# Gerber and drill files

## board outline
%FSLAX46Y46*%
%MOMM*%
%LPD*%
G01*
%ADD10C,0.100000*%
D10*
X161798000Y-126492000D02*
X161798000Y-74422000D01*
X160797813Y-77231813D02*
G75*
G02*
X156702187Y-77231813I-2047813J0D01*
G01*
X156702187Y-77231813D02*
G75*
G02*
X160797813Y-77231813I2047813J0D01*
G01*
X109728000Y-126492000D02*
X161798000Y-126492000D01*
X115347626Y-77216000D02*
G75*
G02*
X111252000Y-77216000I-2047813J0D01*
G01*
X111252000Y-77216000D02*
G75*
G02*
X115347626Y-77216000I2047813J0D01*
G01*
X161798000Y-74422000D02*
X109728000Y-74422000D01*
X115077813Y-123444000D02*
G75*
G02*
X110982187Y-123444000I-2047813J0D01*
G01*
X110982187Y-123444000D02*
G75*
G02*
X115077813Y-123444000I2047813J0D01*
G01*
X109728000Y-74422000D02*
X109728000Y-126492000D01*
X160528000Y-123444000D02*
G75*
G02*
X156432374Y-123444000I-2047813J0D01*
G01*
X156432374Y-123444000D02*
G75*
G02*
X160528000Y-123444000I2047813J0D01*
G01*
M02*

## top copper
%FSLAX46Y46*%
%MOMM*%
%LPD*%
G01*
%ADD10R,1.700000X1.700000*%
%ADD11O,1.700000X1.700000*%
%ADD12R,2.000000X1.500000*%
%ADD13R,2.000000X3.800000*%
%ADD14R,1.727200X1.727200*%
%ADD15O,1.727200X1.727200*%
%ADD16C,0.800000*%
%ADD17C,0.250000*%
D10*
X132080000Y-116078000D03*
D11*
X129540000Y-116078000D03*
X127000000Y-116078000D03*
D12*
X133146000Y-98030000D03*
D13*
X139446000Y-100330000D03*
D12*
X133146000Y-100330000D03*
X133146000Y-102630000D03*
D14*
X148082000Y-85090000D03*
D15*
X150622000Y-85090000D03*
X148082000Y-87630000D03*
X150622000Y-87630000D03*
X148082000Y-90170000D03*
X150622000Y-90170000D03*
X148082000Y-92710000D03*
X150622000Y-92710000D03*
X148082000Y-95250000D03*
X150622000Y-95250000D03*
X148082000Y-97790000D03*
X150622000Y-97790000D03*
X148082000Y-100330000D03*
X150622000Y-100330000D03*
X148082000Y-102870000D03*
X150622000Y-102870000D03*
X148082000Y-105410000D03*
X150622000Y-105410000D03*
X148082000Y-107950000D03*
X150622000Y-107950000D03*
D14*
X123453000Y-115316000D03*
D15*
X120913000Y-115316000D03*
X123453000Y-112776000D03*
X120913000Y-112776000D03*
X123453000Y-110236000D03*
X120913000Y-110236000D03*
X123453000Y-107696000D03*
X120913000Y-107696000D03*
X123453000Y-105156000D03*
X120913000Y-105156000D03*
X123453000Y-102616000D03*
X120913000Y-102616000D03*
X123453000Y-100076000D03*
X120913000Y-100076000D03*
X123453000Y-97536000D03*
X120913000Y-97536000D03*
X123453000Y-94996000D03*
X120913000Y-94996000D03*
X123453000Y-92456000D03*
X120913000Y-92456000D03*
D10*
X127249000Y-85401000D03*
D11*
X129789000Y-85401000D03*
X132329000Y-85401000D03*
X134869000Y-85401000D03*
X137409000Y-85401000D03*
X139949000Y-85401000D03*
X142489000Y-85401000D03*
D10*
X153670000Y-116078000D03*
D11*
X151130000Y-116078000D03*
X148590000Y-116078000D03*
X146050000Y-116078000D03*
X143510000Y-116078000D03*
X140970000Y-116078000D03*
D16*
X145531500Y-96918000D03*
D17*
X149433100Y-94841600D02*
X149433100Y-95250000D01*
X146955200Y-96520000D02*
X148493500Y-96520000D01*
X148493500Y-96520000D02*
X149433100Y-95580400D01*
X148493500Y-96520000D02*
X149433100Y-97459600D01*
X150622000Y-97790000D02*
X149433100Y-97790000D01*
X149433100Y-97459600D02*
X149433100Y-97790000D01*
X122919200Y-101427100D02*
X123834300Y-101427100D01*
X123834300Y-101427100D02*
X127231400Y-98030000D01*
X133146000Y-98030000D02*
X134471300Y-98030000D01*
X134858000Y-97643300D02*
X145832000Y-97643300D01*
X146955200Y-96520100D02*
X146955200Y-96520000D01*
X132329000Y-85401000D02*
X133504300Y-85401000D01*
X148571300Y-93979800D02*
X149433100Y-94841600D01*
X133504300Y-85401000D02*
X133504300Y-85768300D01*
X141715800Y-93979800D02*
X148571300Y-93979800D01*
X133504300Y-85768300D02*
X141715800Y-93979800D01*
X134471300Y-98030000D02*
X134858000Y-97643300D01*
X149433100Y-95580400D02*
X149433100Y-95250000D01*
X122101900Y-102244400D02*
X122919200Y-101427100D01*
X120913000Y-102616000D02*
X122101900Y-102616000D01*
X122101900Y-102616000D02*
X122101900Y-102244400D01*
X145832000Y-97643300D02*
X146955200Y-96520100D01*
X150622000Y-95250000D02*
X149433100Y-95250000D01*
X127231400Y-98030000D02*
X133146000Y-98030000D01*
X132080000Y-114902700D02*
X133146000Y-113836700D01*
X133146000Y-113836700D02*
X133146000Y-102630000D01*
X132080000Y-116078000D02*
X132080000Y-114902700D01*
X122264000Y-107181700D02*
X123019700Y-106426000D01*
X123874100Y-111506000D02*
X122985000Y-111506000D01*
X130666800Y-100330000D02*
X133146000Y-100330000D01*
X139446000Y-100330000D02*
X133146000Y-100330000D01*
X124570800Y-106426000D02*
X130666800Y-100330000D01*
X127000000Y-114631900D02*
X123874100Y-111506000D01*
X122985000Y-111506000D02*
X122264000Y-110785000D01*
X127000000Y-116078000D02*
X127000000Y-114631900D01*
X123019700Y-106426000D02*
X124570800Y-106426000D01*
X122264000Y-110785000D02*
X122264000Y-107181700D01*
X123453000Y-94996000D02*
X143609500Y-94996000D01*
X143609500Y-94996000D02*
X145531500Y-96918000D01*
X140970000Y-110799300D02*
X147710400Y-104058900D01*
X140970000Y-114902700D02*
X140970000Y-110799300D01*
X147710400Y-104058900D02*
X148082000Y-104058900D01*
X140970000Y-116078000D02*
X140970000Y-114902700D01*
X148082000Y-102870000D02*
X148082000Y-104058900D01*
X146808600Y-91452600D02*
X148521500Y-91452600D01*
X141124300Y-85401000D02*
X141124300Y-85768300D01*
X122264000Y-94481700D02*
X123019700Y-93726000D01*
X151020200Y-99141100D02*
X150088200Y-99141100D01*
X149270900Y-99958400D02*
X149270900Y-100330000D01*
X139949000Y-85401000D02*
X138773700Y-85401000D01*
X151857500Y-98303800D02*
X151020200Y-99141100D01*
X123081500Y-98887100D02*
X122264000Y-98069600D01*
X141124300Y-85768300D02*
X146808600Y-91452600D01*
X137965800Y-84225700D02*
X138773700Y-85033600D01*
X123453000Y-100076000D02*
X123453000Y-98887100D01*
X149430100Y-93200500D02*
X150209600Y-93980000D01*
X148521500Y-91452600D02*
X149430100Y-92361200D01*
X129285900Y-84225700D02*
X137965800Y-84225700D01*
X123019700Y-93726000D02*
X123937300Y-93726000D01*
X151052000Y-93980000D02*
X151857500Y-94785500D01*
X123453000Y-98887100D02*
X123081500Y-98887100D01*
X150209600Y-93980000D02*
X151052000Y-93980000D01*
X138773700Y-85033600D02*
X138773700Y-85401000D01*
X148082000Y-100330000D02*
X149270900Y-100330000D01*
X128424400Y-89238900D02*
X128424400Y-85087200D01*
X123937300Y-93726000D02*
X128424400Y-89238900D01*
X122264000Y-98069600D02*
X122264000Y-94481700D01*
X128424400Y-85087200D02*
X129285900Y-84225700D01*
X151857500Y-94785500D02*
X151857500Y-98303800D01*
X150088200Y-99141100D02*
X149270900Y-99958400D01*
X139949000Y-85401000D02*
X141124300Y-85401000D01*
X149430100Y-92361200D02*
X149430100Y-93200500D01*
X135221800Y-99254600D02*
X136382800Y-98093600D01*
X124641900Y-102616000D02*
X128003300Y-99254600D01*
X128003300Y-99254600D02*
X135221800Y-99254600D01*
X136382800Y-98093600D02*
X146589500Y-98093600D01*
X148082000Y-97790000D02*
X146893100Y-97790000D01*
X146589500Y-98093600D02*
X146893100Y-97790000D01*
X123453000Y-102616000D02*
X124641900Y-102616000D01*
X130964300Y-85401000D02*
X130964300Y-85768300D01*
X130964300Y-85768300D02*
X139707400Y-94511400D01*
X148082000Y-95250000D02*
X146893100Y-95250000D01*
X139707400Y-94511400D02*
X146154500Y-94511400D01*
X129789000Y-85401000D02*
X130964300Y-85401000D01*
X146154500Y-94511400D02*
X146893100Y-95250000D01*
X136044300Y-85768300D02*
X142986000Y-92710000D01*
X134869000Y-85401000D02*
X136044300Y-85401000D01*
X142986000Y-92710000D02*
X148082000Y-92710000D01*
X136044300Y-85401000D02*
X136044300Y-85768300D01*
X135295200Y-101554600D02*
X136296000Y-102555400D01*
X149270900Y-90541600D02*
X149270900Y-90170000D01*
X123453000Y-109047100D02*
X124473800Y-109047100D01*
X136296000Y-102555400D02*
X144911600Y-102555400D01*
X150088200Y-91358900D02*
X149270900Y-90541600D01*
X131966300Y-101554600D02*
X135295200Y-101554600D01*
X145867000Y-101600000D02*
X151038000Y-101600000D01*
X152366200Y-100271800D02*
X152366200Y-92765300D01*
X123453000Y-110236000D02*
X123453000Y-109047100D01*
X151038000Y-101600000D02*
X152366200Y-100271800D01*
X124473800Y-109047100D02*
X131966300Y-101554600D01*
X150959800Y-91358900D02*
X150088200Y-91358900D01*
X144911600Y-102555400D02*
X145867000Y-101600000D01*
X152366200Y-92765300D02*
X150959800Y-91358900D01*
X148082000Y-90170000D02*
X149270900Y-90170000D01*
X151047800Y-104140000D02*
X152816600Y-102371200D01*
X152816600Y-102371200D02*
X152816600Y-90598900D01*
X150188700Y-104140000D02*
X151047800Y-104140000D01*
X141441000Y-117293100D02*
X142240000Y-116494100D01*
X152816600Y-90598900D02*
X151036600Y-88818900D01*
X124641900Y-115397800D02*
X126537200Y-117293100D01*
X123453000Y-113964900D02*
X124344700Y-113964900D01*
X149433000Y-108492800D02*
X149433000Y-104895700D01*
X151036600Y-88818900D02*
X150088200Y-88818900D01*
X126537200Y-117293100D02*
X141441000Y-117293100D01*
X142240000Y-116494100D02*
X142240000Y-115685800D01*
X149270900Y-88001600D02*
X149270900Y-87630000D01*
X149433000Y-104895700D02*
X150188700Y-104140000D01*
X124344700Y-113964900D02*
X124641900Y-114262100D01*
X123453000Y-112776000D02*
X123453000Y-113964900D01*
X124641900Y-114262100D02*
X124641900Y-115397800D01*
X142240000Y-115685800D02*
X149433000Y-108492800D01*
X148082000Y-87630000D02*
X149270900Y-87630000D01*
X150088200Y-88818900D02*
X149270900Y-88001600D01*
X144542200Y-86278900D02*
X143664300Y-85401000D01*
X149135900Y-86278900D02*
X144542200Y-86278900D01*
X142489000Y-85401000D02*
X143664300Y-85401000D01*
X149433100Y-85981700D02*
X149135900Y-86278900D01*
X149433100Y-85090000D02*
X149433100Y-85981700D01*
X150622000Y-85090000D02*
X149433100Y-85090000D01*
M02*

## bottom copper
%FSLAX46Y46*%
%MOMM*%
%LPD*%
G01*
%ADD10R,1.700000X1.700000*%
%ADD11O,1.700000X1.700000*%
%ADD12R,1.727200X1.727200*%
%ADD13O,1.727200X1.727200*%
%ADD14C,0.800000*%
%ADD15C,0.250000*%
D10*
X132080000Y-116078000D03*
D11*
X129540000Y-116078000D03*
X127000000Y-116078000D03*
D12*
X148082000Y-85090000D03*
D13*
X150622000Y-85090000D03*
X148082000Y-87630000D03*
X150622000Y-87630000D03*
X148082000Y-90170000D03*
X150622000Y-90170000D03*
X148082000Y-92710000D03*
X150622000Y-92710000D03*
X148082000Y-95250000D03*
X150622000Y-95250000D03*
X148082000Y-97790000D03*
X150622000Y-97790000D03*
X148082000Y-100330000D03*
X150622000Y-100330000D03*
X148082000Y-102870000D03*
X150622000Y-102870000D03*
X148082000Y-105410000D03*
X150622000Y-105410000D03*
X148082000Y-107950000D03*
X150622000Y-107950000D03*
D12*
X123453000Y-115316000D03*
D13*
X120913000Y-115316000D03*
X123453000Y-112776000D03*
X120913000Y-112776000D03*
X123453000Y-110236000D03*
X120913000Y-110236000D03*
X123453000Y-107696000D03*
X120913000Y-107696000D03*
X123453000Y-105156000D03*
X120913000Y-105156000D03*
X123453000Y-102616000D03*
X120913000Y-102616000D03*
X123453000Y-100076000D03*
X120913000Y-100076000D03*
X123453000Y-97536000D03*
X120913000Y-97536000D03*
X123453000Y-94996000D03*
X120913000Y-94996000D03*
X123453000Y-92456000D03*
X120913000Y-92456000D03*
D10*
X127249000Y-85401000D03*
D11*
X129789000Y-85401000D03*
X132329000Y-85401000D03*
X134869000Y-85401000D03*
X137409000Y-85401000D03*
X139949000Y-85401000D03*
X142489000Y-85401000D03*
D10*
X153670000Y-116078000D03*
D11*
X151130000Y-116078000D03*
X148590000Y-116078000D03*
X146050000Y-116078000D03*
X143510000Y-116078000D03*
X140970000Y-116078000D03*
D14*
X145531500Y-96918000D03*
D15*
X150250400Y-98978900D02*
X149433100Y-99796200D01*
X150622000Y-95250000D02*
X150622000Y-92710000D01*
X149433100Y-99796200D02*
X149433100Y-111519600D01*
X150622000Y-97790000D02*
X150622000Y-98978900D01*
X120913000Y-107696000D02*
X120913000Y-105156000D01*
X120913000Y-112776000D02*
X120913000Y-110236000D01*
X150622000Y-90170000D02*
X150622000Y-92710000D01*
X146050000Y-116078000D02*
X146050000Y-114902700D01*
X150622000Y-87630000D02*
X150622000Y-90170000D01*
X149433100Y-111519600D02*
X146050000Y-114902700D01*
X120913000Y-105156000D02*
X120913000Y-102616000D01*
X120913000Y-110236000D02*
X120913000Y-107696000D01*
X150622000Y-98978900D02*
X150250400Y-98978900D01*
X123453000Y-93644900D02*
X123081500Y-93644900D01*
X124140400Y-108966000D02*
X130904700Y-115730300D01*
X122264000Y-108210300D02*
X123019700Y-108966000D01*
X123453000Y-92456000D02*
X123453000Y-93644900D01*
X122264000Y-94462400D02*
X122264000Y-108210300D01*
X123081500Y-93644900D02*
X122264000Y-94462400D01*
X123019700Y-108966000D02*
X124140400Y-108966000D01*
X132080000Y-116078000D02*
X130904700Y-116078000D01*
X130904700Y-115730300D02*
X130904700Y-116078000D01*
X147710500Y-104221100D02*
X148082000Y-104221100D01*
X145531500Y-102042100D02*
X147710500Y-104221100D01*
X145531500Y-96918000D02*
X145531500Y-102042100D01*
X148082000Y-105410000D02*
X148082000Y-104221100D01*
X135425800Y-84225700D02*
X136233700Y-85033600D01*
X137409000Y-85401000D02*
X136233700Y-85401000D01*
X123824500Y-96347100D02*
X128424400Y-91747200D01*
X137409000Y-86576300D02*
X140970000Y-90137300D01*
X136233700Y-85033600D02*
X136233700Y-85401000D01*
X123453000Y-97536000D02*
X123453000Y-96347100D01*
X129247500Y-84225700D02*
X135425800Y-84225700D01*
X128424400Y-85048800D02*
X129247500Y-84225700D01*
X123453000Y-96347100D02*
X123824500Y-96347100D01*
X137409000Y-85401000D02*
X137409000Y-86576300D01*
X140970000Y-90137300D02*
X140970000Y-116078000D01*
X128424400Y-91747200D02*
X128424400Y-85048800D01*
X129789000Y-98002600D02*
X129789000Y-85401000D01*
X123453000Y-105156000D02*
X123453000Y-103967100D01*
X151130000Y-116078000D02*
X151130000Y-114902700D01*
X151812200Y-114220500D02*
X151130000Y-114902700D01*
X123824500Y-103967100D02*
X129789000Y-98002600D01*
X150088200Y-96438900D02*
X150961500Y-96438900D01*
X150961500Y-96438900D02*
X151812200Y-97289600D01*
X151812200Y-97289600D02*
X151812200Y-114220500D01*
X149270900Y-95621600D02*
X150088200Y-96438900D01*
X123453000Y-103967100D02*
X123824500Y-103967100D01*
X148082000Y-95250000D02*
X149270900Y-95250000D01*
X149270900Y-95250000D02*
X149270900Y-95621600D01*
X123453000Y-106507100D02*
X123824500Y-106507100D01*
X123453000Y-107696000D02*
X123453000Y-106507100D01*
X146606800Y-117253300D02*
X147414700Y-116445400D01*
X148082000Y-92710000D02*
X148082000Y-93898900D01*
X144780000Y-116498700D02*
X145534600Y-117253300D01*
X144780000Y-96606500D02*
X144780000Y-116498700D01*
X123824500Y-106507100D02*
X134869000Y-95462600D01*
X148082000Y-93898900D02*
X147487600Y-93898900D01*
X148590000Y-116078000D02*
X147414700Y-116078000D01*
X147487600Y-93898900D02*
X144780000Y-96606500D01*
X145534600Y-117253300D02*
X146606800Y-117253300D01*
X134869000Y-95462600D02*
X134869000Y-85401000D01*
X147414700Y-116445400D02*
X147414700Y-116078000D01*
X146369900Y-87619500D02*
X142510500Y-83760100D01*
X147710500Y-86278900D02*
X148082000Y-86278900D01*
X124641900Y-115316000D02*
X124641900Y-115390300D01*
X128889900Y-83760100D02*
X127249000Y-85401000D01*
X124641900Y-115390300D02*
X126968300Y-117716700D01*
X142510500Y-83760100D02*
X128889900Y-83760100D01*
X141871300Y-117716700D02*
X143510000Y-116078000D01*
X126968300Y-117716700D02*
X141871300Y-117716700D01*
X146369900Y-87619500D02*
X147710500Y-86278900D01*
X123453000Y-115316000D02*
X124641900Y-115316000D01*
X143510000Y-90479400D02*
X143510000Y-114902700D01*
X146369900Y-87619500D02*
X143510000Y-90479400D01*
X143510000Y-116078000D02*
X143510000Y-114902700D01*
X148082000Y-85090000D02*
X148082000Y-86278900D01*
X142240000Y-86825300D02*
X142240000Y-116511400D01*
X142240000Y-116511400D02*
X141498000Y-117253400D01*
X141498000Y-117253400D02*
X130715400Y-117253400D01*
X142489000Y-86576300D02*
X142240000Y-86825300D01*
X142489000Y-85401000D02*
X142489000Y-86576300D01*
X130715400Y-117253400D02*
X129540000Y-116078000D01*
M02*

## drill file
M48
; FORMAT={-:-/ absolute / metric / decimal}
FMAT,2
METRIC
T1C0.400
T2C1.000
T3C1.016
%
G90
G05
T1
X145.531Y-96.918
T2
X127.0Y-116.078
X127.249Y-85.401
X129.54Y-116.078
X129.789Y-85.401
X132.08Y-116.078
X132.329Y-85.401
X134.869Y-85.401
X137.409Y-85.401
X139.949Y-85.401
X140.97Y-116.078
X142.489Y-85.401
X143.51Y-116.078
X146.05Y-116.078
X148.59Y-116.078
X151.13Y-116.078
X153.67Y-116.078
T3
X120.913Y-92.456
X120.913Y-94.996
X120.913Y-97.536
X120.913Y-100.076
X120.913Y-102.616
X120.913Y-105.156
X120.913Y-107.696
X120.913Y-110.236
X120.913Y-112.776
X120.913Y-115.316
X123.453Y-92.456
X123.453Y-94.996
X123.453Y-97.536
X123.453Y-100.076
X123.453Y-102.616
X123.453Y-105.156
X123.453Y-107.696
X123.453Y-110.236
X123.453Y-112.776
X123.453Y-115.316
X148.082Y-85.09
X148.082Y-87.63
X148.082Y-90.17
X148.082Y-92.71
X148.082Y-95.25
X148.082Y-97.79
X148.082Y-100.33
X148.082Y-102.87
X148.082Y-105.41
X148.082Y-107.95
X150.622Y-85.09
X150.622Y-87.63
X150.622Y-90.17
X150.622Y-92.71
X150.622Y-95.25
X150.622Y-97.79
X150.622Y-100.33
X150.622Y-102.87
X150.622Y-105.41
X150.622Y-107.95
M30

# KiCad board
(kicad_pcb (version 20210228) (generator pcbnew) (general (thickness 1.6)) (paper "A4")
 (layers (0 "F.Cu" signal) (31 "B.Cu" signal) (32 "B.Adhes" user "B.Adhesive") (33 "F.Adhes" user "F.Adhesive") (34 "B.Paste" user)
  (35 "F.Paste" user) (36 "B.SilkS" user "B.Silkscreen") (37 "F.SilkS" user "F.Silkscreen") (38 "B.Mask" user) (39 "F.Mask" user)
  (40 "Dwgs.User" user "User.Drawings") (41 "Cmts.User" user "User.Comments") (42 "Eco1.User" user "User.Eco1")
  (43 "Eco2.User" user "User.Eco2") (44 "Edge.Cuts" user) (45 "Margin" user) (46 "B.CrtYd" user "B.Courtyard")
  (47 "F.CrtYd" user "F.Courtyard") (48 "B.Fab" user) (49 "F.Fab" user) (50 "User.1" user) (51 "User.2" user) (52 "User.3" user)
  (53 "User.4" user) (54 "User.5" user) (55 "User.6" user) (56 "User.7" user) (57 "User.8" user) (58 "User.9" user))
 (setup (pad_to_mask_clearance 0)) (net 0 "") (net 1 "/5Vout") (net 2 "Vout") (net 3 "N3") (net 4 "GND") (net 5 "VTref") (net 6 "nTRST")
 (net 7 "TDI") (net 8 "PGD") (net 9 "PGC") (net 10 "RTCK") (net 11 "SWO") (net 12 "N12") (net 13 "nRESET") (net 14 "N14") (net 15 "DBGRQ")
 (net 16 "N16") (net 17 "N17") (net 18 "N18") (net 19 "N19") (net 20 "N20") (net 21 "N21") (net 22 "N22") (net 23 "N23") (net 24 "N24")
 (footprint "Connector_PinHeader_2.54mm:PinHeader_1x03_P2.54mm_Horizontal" (layer "F.Cu") (at 132.08 116.078 -90)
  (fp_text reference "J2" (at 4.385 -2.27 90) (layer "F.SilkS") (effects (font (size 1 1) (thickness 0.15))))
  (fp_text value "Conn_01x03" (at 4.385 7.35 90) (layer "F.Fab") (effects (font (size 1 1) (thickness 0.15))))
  (pad "1" thru_hole rect (at 0 0 270) (locked) (size 1.7 1.7) (drill 1) (layers *.Cu *.Mask) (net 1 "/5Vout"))
  (pad "2" thru_hole oval (at 0 2.54 270) (locked) (size 1.7 1.7) (drill 1) (layers *.Cu *.Mask) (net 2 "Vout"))
  (pad "3" thru_hole oval (at 0 5.08 270) (locked) (size 1.7 1.7) (drill 1) (layers *.Cu *.Mask) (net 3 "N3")))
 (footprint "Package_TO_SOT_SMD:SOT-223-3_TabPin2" (layer "F.Cu") (at 136.296 100.33)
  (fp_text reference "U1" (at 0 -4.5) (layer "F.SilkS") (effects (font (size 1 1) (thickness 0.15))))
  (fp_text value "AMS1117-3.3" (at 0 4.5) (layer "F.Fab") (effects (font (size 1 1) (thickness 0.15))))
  (pad "1" smd rect (at -3.15 -2.3) (locked) (size 2 1.5) (layers "F.Cu" "F.Paste" "F.Mask") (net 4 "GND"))
  (pad "2" smd rect (at 3.15 0) (locked) (size 2 3.8) (layers "F.Cu" "F.Paste" "F.Mask") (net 3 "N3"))
  (pad "2" smd rect (at -3.15 0) (locked) (size 2 1.5) (layers "F.Cu" "F.Paste" "F.Mask") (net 3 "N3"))
  (pad "3" smd rect (at -3.15 2.3) (locked) (size 2 1.5) (layers "F.Cu" "F.Paste" "F.Mask") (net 1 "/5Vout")))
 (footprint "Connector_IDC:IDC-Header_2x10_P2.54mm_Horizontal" (layer "F.Cu") (at 148.082 85.09)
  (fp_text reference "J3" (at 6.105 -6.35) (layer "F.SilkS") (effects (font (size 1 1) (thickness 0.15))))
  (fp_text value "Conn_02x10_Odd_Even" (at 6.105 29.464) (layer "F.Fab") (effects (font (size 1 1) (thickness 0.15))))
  (pad "1" thru_hole rect (at 0 0) (locked) (size 1.7272 1.7272) (drill 1.016) (layers *.Cu *.Mask) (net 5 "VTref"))
  (pad "2" thru_hole oval (at 2.54 0) (locked) (size 1.7272 1.7272) (drill 1.016) (layers *.Cu *.Mask) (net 2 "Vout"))
  (pad "3" thru_hole oval (at 0 2.54) (locked) (size 1.7272 1.7272) (drill 1.016) (layers *.Cu *.Mask) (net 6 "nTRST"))
  (pad "4" thru_hole oval (at 2.54 2.54) (locked) (size 1.7272 1.7272) (drill 1.016) (layers *.Cu *.Mask) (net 4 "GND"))
  (pad "5" thru_hole oval (at 0 5.08) (locked) (size 1.7272 1.7272) (drill 1.016) (layers *.Cu *.Mask) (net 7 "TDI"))
  (pad "6" thru_hole oval (at 2.54 5.08) (locked) (size 1.7272 1.7272) (drill 1.016) (layers *.Cu *.Mask) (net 4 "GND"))
  (pad "7" thru_hole oval (at 0 7.62) (locked) (size 1.7272 1.7272) (drill 1.016) (layers *.Cu *.Mask) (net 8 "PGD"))
  (pad "8" thru_hole oval (at 2.54 7.62) (locked) (size 1.7272 1.7272) (drill 1.016) (layers *.Cu *.Mask) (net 4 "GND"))
  (pad "9" thru_hole oval (at 0 10.16) (locked) (size 1.7272 1.7272) (drill 1.016) (layers *.Cu *.Mask) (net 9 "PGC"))
  (pad "10" thru_hole oval (at 2.54 10.16) (locked) (size 1.7272 1.7272) (drill 1.016) (layers *.Cu *.Mask) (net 4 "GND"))
  (pad "11" thru_hole oval (at 0 12.7) (locked) (size 1.7272 1.7272) (drill 1.016) (layers *.Cu *.Mask) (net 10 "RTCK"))
  (pad "12" thru_hole oval (at 2.54 12.7) (locked) (size 1.7272 1.7272) (drill 1.016) (layers *.Cu *.Mask) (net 4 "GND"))
  (pad "13" thru_hole oval (at 0 15.24) (locked) (size 1.7272 1.7272) (drill 1.016) (layers *.Cu *.Mask) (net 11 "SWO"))
  (pad "14" thru_hole oval (at 2.54 15.24) (locked) (size 1.7272 1.7272) (drill 1.016) (layers *.Cu *.Mask) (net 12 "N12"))
  (pad "15" thru_hole oval (at 0 17.78) (locked) (size 1.7272 1.7272) (drill 1.016) (layers *.Cu *.Mask) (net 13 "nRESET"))
  (pad "16" thru_hole oval (at 2.54 17.78) (locked) (size 1.7272 1.7272) (drill 1.016) (layers *.Cu *.Mask) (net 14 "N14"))
  (pad "17" thru_hole oval (at 0 20.32) (locked) (size 1.7272 1.7272) (drill 1.016) (layers *.Cu *.Mask) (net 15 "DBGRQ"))
  (pad "18" thru_hole oval (at 2.54 20.32) (locked) (size 1.7272 1.7272) (drill 1.016) (layers *.Cu *.Mask) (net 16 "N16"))
  (pad "19" thru_hole oval (at 0 22.86) (locked) (size 1.7272 1.7272) (drill 1.016) (layers *.Cu *.Mask) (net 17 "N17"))
  (pad "20" thru_hole oval (at 2.54 22.86) (locked) (size 1.7272 1.7272) (drill 1.016) (layers *.Cu *.Mask) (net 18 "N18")))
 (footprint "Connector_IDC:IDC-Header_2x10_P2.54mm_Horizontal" (layer "F.Cu") (at 123.453 115.316 180)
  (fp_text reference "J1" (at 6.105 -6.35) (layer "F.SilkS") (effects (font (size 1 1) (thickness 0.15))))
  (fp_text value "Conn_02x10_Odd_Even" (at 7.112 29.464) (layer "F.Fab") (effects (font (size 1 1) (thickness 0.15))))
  (pad "1" thru_hole rect (at 0 0 180) (locked) (size 1.7272 1.7272) (drill 1.016) (layers *.Cu *.Mask) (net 5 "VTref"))
  (pad "2" thru_hole oval (at 2.54 0 180) (locked) (size 1.7272 1.7272) (drill 1.016) (layers *.Cu *.Mask) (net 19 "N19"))
  (pad "3" thru_hole oval (at 0 2.54 180) (locked) (size 1.7272 1.7272) (drill 1.016) (layers *.Cu *.Mask) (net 6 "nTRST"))
  (pad "4" thru_hole oval (at 2.54 2.54 180) (locked) (size 1.7272 1.7272) (drill 1.016) (layers *.Cu *.Mask) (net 4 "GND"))
  (pad "5" thru_hole oval (at 0 5.08 180) (locked) (size 1.7272 1.7272) (drill 1.016) (layers *.Cu *.Mask) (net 7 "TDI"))
  (pad "6" thru_hole oval (at 2.54 5.08 180) (locked) (size 1.7272 1.7272) (drill 1.016) (layers *.Cu *.Mask) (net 4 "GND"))
  (pad "7" thru_hole oval (at 0 7.62 180) (locked) (size 1.7272 1.7272) (drill 1.016) (layers *.Cu *.Mask) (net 8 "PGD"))
  (pad "8" thru_hole oval (at 2.54 7.62 180) (locked) (size 1.7272 1.7272) (drill 1.016) (layers *.Cu *.Mask) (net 4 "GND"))
  (pad "9" thru_hole oval (at 0 10.16 180) (locked) (size 1.7272 1.7272) (drill 1.016) (layers *.Cu *.Mask) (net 9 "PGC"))
  (pad "10" thru_hole oval (at 2.54 10.16 180) (locked) (size 1.7272 1.7272) (drill 1.016) (layers *.Cu *.Mask) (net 4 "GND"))
  (pad "11" thru_hole oval (at 0 12.7 180) (locked) (size 1.7272 1.7272) (drill 1.016) (layers *.Cu *.Mask) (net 10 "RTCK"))
  (pad "12" thru_hole oval (at 2.54 12.7 180) (locked) (size 1.7272 1.7272) (drill 1.016) (layers *.Cu *.Mask) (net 4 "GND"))
  (pad "13" thru_hole oval (at 0 15.24 180) (locked) (size 1.7272 1.7272) (drill 1.016) (layers *.Cu *.Mask) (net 11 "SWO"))
  (pad "14" thru_hole oval (at 2.54 15.24 180) (locked) (size 1.7272 1.7272) (drill 1.016) (layers *.Cu *.Mask) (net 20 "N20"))
  (pad "15" thru_hole oval (at 0 17.78 180) (locked) (size 1.7272 1.7272) (drill 1.016) (layers *.Cu *.Mask) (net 13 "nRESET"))
  (pad "16" thru_hole oval (at 2.54 17.78 180) (locked) (size 1.7272 1.7272) (drill 1.016) (layers *.Cu *.Mask) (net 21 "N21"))
  (pad "17" thru_hole oval (at 0 20.32 180) (locked) (size 1.7272 1.7272) (drill 1.016) (layers *.Cu *.Mask) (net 15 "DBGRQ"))
  (pad "18" thru_hole oval (at 2.54 20.32 180) (locked) (size 1.7272 1.7272) (drill 1.016) (layers *.Cu *.Mask) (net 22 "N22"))
  (pad "19" thru_hole oval (at 0 22.86 180) (locked) (size 1.7272 1.7272) (drill 1.016) (layers *.Cu *.Mask) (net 1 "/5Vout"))
  (pad "20" thru_hole oval (at 2.54 22.86 180) (locked) (size 1.7272 1.7272) (drill 1.016) (layers *.Cu *.Mask) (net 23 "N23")))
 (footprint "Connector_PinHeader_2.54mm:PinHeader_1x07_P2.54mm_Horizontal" (layer "F.Cu") (at 127.249 85.401 90)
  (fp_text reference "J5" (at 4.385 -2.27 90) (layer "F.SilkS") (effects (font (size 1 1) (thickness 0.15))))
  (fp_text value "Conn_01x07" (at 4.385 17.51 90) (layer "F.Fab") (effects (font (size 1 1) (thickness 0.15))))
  (pad "1" thru_hole rect (at 0 0 90) (locked) (size 1.7 1.7) (drill 1) (layers *.Cu *.Mask) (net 5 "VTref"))
  (pad "2" thru_hole oval (at 0 2.54 90) (locked) (size 1.7 1.7) (drill 1) (layers *.Cu *.Mask) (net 9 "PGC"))
  (pad "3" thru_hole oval (at 0 5.08 90) (locked) (size 1.7 1.7) (drill 1) (layers *.Cu *.Mask) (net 4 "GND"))
  (pad "4" thru_hole oval (at 0 7.62 90) (locked) (size 1.7 1.7) (drill 1) (layers *.Cu *.Mask) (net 8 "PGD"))
  (pad "5" thru_hole oval (at 0 10.16 90) (locked) (size 1.7 1.7) (drill 1) (layers *.Cu *.Mask) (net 13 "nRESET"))
  (pad "6" thru_hole oval (at 0 12.7 90) (locked) (size 1.7 1.7) (drill 1) (layers *.Cu *.Mask) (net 11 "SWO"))
  (pad "7" thru_hole oval (at 0 15.24 90) (locked) (size 1.7 1.7) (drill 1) (layers *.Cu *.Mask) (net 2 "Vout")))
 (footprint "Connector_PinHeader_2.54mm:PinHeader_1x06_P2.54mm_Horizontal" (layer "F.Cu") (at 153.67 116.078 -90)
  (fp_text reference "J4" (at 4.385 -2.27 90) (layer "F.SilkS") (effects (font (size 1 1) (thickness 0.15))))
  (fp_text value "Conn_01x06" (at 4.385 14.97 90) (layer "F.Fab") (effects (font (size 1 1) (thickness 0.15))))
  (pad "1" thru_hole rect (at 0 0 270) (locked) (size 1.7 1.7) (drill 1) (layers *.Cu *.Mask) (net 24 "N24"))
  (pad "2" thru_hole oval (at 0 2.54 270) (locked) (size 1.7 1.7) (drill 1) (layers *.Cu *.Mask) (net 9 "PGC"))
  (pad "3" thru_hole oval (at 0 5.08 270) (locked) (size 1.7 1.7) (drill 1) (layers *.Cu *.Mask) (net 8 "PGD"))
  (pad "4" thru_hole oval (at 0 7.62 270) (locked) (size 1.7 1.7) (drill 1) (layers *.Cu *.Mask) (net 4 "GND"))
  (pad "5" thru_hole oval (at 0 10.16 270) (locked) (size 1.7 1.7) (drill 1) (layers *.Cu *.Mask) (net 5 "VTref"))
  (pad "6" thru_hole oval (at 0 12.7 270) (locked) (size 1.7 1.7) (drill 1) (layers *.Cu *.Mask) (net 13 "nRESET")))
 (gr_line (start 161.798 126.492) (end 161.798 74.422) (layer "Edge.Cuts") (width 0.1))
 (gr_circle (center 158.75 77.231813) (end 160.528 78.247813) (layer "Edge.Cuts") (width 0.1) (fill none))
 (gr_line (start 109.728 126.492) (end 161.798 126.492) (layer "Edge.Cuts") (width 0.1))
 (gr_circle (center 113.299813 77.216) (end 115.077813 78.232) (layer "Edge.Cuts") (width 0.1) (fill none))
 (gr_line (start 161.798 74.422) (end 109.728 74.422) (layer "Edge.Cuts") (width 0.1))
 (gr_circle (center 113.03 123.444) (end 114.808 124.46) (layer "Edge.Cuts") (width 0.1) (fill none))
 (gr_line (start 109.728 74.422) (end 109.728 126.492) (layer "Edge.Cuts") (width 0.1))
 (gr_circle (center 158.480187 123.444) (end 160.258187 124.46) (layer "Edge.Cuts") (width 0.1) (fill none))
 (segment (start 149.4331 94.8416) (end 149.4331 95.25) (width 0.25) (layer "F.Cu") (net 4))
 (segment (start 146.9552 96.52) (end 148.4935 96.52) (width 0.25) (layer "F.Cu") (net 4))
 (segment (start 148.4935 96.52) (end 149.4331 95.5804) (width 0.25) (layer "F.Cu") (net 4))
 (segment (start 148.4935 96.52) (end 149.4331 97.4596) (width 0.25) (layer "F.Cu") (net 4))
 (segment (start 150.622 97.79) (end 149.4331 97.79) (width 0.25) (layer "F.Cu") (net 4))
 (segment (start 149.4331 97.4596) (end 149.4331 97.79) (width 0.25) (layer "F.Cu") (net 4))
 (segment (start 122.9192 101.4271) (end 123.8343 101.4271) (width 0.25) (layer "F.Cu") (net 4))
 (segment (start 123.8343 101.4271) (end 127.2314 98.03) (width 0.25) (layer "F.Cu") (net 4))
 (segment (start 133.146 98.03) (end 134.4713 98.03) (width 0.25) (layer "F.Cu") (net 4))
 (segment (start 134.858 97.6433) (end 145.832 97.6433) (width 0.25) (layer "F.Cu") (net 4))
 (segment (start 146.9552 96.5201) (end 146.9552 96.52) (width 0.25) (layer "F.Cu") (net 4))
 (segment (start 132.329 85.401) (end 133.5043 85.401) (width 0.25) (layer "F.Cu") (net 4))
 (segment (start 148.5713 93.9798) (end 149.4331 94.8416) (width 0.25) (layer "F.Cu") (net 4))
 (segment (start 133.5043 85.401) (end 133.5043 85.7683) (width 0.25) (layer "F.Cu") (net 4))
 (segment (start 141.7158 93.9798) (end 148.5713 93.9798) (width 0.25) (layer "F.Cu") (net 4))
 (segment (start 133.5043 85.7683) (end 141.7158 93.9798) (width 0.25) (layer "F.Cu") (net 4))
 (segment (start 134.4713 98.03) (end 134.858 97.6433) (width 0.25) (layer "F.Cu") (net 4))
 (segment (start 149.4331 95.5804) (end 149.4331 95.25) (width 0.25) (layer "F.Cu") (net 4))
 (segment (start 122.1019 102.2444) (end 122.9192 101.4271) (width 0.25) (layer "F.Cu") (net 4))
 (segment (start 120.913 102.616) (end 122.1019 102.616) (width 0.25) (layer "F.Cu") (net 4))
 (segment (start 122.1019 102.616) (end 122.1019 102.2444) (width 0.25) (layer "F.Cu") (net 4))
 (segment (start 145.832 97.6433) (end 146.9552 96.5201) (width 0.25) (layer "F.Cu") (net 4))
 (segment (start 150.622 95.25) (end 149.4331 95.25) (width 0.25) (layer "F.Cu") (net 4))
 (segment (start 127.2314 98.03) (end 133.146 98.03) (width 0.25) (layer "F.Cu") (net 4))
 (segment (start 150.2504 98.9789) (end 149.4331 99.7962) (width 0.25) (layer "B.Cu") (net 4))
 (segment (start 150.622 95.25) (end 150.622 92.71) (width 0.25) (layer "B.Cu") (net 4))
 (segment (start 149.4331 99.7962) (end 149.4331 111.5196) (width 0.25) (layer "B.Cu") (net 4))
 (segment (start 150.622 97.79) (end 150.622 98.9789) (width 0.25) (layer "B.Cu") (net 4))
 (segment (start 120.913 107.696) (end 120.913 105.156) (width 0.25) (layer "B.Cu") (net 4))
 (segment (start 120.913 112.776) (end 120.913 110.236) (width 0.25) (layer "B.Cu") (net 4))
 (segment (start 150.622 90.17) (end 150.622 92.71) (width 0.25) (layer "B.Cu") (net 4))
 (segment (start 146.05 116.078) (end 146.05 114.9027) (width 0.25) (layer "B.Cu") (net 4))
 (segment (start 150.622 87.63) (end 150.622 90.17) (width 0.25) (layer "B.Cu") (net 4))
 (segment (start 149.4331 111.5196) (end 146.05 114.9027) (width 0.25) (layer "B.Cu") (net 4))
 (segment (start 120.913 105.156) (end 120.913 102.616) (width 0.25) (layer "B.Cu") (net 4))
 (segment (start 120.913 110.236) (end 120.913 107.696) (width 0.25) (layer "B.Cu") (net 4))
 (segment (start 150.622 98.9789) (end 150.2504 98.9789) (width 0.25) (layer "B.Cu") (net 4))
 (segment (start 132.08 114.9027) (end 133.146 113.8367) (width 0.25) (layer "F.Cu") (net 1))
 (segment (start 133.146 113.8367) (end 133.146 102.63) (width 0.25) (layer "F.Cu") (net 1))
 (segment (start 132.08 116.078) (end 132.08 114.9027) (width 0.25) (layer "F.Cu") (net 1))
 (segment (start 123.453 93.6449) (end 123.0815 93.6449) (width 0.25) (layer "B.Cu") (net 1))
 (segment (start 124.1404 108.966) (end 130.9047 115.7303) (width 0.25) (layer "B.Cu") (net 1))
 (segment (start 122.264 108.2103) (end 123.0197 108.966) (width 0.25) (layer "B.Cu") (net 1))
 (segment (start 123.453 92.456) (end 123.453 93.6449) (width 0.25) (layer "B.Cu") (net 1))
 (segment (start 122.264 94.4624) (end 122.264 108.2103) (width 0.25) (layer "B.Cu") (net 1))
 (segment (start 123.0815 93.6449) (end 122.264 94.4624) (width 0.25) (layer "B.Cu") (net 1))
 (segment (start 123.0197 108.966) (end 124.1404 108.966) (width 0.25) (layer "B.Cu") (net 1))
 (segment (start 132.08 116.078) (end 130.9047 116.078) (width 0.25) (layer "B.Cu") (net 1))
 (segment (start 130.9047 115.7303) (end 130.9047 116.078) (width 0.25) (layer "B.Cu") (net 1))
 (segment (start 122.264 107.1817) (end 123.0197 106.426) (width 0.25) (layer "F.Cu") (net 3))
 (segment (start 123.8741 111.506) (end 122.985 111.506) (width 0.25) (layer "F.Cu") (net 3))
 (segment (start 130.6668 100.33) (end 133.146 100.33) (width 0.25) (layer "F.Cu") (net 3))
 (segment (start 139.446 100.33) (end 133.146 100.33) (width 0.25) (layer "F.Cu") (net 3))
 (segment (start 124.5708 106.426) (end 130.6668 100.33) (width 0.25) (layer "F.Cu") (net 3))
 (segment (start 127 114.6319) (end 123.8741 111.506) (width 0.25) (layer "F.Cu") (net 3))
 (segment (start 122.985 111.506) (end 122.264 110.785) (width 0.25) (layer "F.Cu") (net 3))
 (segment (start 127 116.078) (end 127 114.6319) (width 0.25) (layer "F.Cu") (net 3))
 (segment (start 123.0197 106.426) (end 124.5708 106.426) (width 0.25) (layer "F.Cu") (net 3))
 (segment (start 122.264 110.785) (end 122.264 107.1817) (width 0.25) (layer "F.Cu") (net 3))
 (segment (start 123.453 94.996) (end 143.6095 94.996) (width 0.25) (layer "F.Cu") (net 15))
 (segment (start 143.6095 94.996) (end 145.5315 96.918) (width 0.25) (layer "F.Cu") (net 15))
 (via (at 145.5315 96.918) (size 0.8) (drill 0.4) (layers "F.Cu" "B.Cu") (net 15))
 (segment (start 147.7105 104.2211) (end 148.082 104.2211) (width 0.25) (layer "B.Cu") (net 15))
 (segment (start 145.5315 102.0421) (end 147.7105 104.2211) (width 0.25) (layer "B.Cu") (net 15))
 (segment (start 145.5315 96.918) (end 145.5315 102.0421) (width 0.25) (layer "B.Cu") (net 15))
 (segment (start 148.082 105.41) (end 148.082 104.2211) (width 0.25) (layer "B.Cu") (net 15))
 (segment (start 140.97 110.7993) (end 147.7104 104.0589) (width 0.25) (layer "F.Cu") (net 13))
 (segment (start 140.97 114.9027) (end 140.97 110.7993) (width 0.25) (layer "F.Cu") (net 13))
 (segment (start 147.7104 104.0589) (end 148.082 104.0589) (width 0.25) (layer "F.Cu") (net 13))
 (segment (start 140.97 116.078) (end 140.97 114.9027) (width 0.25) (layer "F.Cu") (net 13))
 (segment (start 148.082 102.87) (end 148.082 104.0589) (width 0.25) (layer "F.Cu") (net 13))
 (segment (start 135.4258 84.2257) (end 136.2337 85.0336) (width 0.25) (layer "B.Cu") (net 13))
 (segment (start 137.409 85.401) (end 136.2337 85.401) (width 0.25) (layer "B.Cu") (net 13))
 (segment (start 123.8245 96.3471) (end 128.4244 91.7472) (width 0.25) (layer "B.Cu") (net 13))
 (segment (start 137.409 86.5763) (end 140.97 90.1373) (width 0.25) (layer "B.Cu") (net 13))
 (segment (start 136.2337 85.0336) (end 136.2337 85.401) (width 0.25) (layer "B.Cu") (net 13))
 (segment (start 123.453 97.536) (end 123.453 96.3471) (width 0.25) (layer "B.Cu") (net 13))
 (segment (start 129.2475 84.2257) (end 135.4258 84.2257) (width 0.25) (layer "B.Cu") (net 13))
 (segment (start 128.4244 85.0488) (end 129.2475 84.2257) (width 0.25) (layer "B.Cu") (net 13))
 (segment (start 123.453 96.3471) (end 123.8245 96.3471) (width 0.25) (layer "B.Cu") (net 13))
 (segment (start 137.409 85.401) (end 137.409 86.5763) (width 0.25) (layer "B.Cu") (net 13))
 (segment (start 140.97 90.1373) (end 140.97 116.078) (width 0.25) (layer "B.Cu") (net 13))
 (segment (start 128.4244 91.7472) (end 128.4244 85.0488) (width 0.25) (layer "B.Cu") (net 13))
 (segment (start 146.8086 91.4526) (end 148.5215 91.4526) (width 0.25) (layer "F.Cu") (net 11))
 (segment (start 141.1243 85.401) (end 141.1243 85.7683) (width 0.25) (layer "F.Cu") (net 11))
 (segment (start 122.264 94.4817) (end 123.0197 93.726) (width 0.25) (layer "F.Cu") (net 11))
 (segment (start 151.0202 99.1411) (end 150.0882 99.1411) (width 0.25) (layer "F.Cu") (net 11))
 (segment (start 149.2709 99.9584) (end 149.2709 100.33) (width 0.25) (layer "F.Cu") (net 11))
 (segment (start 139.949 85.401) (end 138.7737 85.401) (width 0.25) (layer "F.Cu") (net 11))
 (segment (start 151.8575 98.3038) (end 151.0202 99.1411) (width 0.25) (layer "F.Cu") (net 11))
 (segment (start 123.0815 98.8871) (end 122.264 98.0696) (width 0.25) (layer "F.Cu") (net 11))
 (segment (start 141.1243 85.7683) (end 146.8086 91.4526) (width 0.25) (layer "F.Cu") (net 11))
 (segment (start 137.9658 84.2257) (end 138.7737 85.0336) (width 0.25) (layer "F.Cu") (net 11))
 (segment (start 123.453 100.076) (end 123.453 98.8871) (width 0.25) (layer "F.Cu") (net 11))
 (segment (start 149.4301 93.2005) (end 150.2096 93.98) (width 0.25) (layer "F.Cu") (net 11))
 (segment (start 148.5215 91.4526) (end 149.4301 92.3612) (width 0.25) (layer "F.Cu") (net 11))
 (segment (start 129.2859 84.2257) (end 137.9658 84.2257) (width 0.25) (layer "F.Cu") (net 11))
 (segment (start 123.0197 93.726) (end 123.9373 93.726) (width 0.25) (layer "F.Cu") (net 11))
 (segment (start 151.052 93.98) (end 151.8575 94.7855) (width 0.25) (layer "F.Cu") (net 11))
 (segment (start 123.453 98.8871) (end 123.0815 98.8871) (width 0.25) (layer "F.Cu") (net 11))
 (segment (start 150.2096 93.98) (end 151.052 93.98) (width 0.25) (layer "F.Cu") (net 11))
 (segment (start 138.7737 85.0336) (end 138.7737 85.401) (width 0.25) (layer "F.Cu") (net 11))
 (segment (start 148.082 100.33) (end 149.2709 100.33) (width 0.25) (layer "F.Cu") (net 11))
 (segment (start 128.4244 89.2389) (end 128.4244 85.0872) (width 0.25) (layer "F.Cu") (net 11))
 (segment (start 123.9373 93.726) (end 128.4244 89.2389) (width 0.25) (layer "F.Cu") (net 11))
 (segment (start 122.264 98.0696) (end 122.264 94.4817) (width 0.25) (layer "F.Cu") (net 11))
 (segment (start 128.4244 85.0872) (end 129.2859 84.2257) (width 0.25) (layer "F.Cu") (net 11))
 (segment (start 151.8575 94.7855) (end 151.8575 98.3038) (width 0.25) (layer "F.Cu") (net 11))
 (segment (start 150.0882 99.1411) (end 149.2709 99.9584) (width 0.25) (layer "F.Cu") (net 11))
 (segment (start 139.949 85.401) (end 141.1243 85.401) (width 0.25) (layer "F.Cu") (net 11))
 (segment (start 149.4301 92.3612) (end 149.4301 93.2005) (width 0.25) (layer "F.Cu") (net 11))
 (segment (start 135.2218 99.2546) (end 136.3828 98.0936) (width 0.25) (layer "F.Cu") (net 10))
 (segment (start 124.6419 102.616) (end 128.0033 99.2546) (width 0.25) (layer "F.Cu") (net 10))
 (segment (start 128.0033 99.2546) (end 135.2218 99.2546) (width 0.25) (layer "F.Cu") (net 10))
 (segment (start 136.3828 98.0936) (end 146.5895 98.0936) (width 0.25) (layer "F.Cu") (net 10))
 (segment (start 148.082 97.79) (end 146.8931 97.79) (width 0.25) (layer "F.Cu") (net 10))
 (segment (start 146.5895 98.0936) (end 146.8931 97.79) (width 0.25) (layer "F.Cu") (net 10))
 (segment (start 123.453 102.616) (end 124.6419 102.616) (width 0.25) (layer "F.Cu") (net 10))
 (segment (start 130.9643 85.401) (end 130.9643 85.7683) (width 0.25) (layer "F.Cu") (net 9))
 (segment (start 130.9643 85.7683) (end 139.7074 94.5114) (width 0.25) (layer "F.Cu") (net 9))
 (segment (start 148.082 95.25) (end 146.8931 95.25) (width 0.25) (layer "F.Cu") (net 9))
 (segment (start 139.7074 94.5114) (end 146.1545 94.5114) (width 0.25) (layer "F.Cu") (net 9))
 (segment (start 129.789 85.401) (end 130.9643 85.401) (width 0.25) (layer "F.Cu") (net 9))
 (segment (start 146.1545 94.5114) (end 146.8931 95.25) (width 0.25) (layer "F.Cu") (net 9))
 (segment (start 129.789 98.0026) (end 129.789 85.401) (width 0.25) (layer "B.Cu") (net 9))
 (segment (start 123.453 105.156) (end 123.453 103.9671) (width 0.25) (layer "B.Cu") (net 9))
 (segment (start 151.13 116.078) (end 151.13 114.9027) (width 0.25) (layer "B.Cu") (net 9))
 (segment (start 151.8122 114.2205) (end 151.13 114.9027) (width 0.25) (layer "B.Cu") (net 9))
 (segment (start 123.8245 103.9671) (end 129.789 98.0026) (width 0.25) (layer "B.Cu") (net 9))
 (segment (start 150.0882 96.4389) (end 150.9615 96.4389) (width 0.25) (layer "B.Cu") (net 9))
 (segment (start 150.9615 96.4389) (end 151.8122 97.2896) (width 0.25) (layer "B.Cu") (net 9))
 (segment (start 151.8122 97.2896) (end 151.8122 114.2205) (width 0.25) (layer "B.Cu") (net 9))
 (segment (start 149.2709 95.6216) (end 150.0882 96.4389) (width 0.25) (layer "B.Cu") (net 9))
 (segment (start 123.453 103.9671) (end 123.8245 103.9671) (width 0.25) (layer "B.Cu") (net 9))
 (segment (start 148.082 95.25) (end 149.2709 95.25) (width 0.25) (layer "B.Cu") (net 9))
 (segment (start 149.2709 95.25) (end 149.2709 95.6216) (width 0.25) (layer "B.Cu") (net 9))
 (segment (start 136.0443 85.7683) (end 142.986 92.71) (width 0.25) (layer "F.Cu") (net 8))
 (segment (start 134.869 85.401) (end 136.0443 85.401) (width 0.25) (layer "F.Cu") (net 8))
 (segment (start 142.986 92.71) (end 148.082 92.71) (width 0.25) (layer "F.Cu") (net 8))
 (segment (start 136.0443 85.401) (end 136.0443 85.7683) (width 0.25) (layer "F.Cu") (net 8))
 (segment (start 123.453 106.5071) (end 123.8245 106.5071) (width 0.25) (layer "B.Cu") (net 8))
 (segment (start 123.453 107.696) (end 123.453 106.5071) (width 0.25) (layer "B.Cu") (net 8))
 (segment (start 146.6068 117.2533) (end 147.4147 116.4454) (width 0.25) (layer "B.Cu") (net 8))
 (segment (start 148.082 92.71) (end 148.082 93.8989) (width 0.25) (layer "B.Cu") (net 8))
 (segment (start 144.78 116.4987) (end 145.5346 117.2533) (width 0.25) (layer "B.Cu") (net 8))
 (segment (start 144.78 96.6065) (end 144.78 116.4987) (width 0.25) (layer "B.Cu") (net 8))
 (segment (start 123.8245 106.5071) (end 134.869 95.4626) (width 0.25) (layer "B.Cu") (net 8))
 (segment (start 148.082 93.8989) (end 147.4876 93.8989) (width 0.25) (layer "B.Cu") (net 8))
 (segment (start 148.59 116.078) (end 147.4147 116.078) (width 0.25) (layer "B.Cu") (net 8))
 (segment (start 147.4876 93.8989) (end 144.78 96.6065) (width 0.25) (layer "B.Cu") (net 8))
 (segment (start 145.5346 117.2533) (end 146.6068 117.2533) (width 0.25) (layer "B.Cu") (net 8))
 (segment (start 134.869 95.4626) (end 134.869 85.401) (width 0.25) (layer "B.Cu") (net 8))
 (segment (start 147.4147 116.4454) (end 147.4147 116.078) (width 0.25) (layer "B.Cu") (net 8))
 (segment (start 135.2952 101.5546) (end 136.296 102.5554) (width 0.25) (layer "F.Cu") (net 7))
 (segment (start 149.2709 90.5416) (end 149.2709 90.17) (width 0.25) (layer "F.Cu") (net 7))
 (segment (start 123.453 109.0471) (end 124.4738 109.0471) (width 0.25) (layer "F.Cu") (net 7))
 (segment (start 136.296 102.5554) (end 144.9116 102.5554) (width 0.25) (layer "F.Cu") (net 7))
 (segment (start 150.0882 91.3589) (end 149.2709 90.5416) (width 0.25) (layer "F.Cu") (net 7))
 (segment (start 131.9663 101.5546) (end 135.2952 101.5546) (width 0.25) (layer "F.Cu") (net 7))
 (segment (start 145.867 101.6) (end 151.038 101.6) (width 0.25) (layer "F.Cu") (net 7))
 (segment (start 152.3662 100.2718) (end 152.3662 92.7653) (width 0.25) (layer "F.Cu") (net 7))
 (segment (start 123.453 110.236) (end 123.453 109.0471) (width 0.25) (layer "F.Cu") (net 7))
 (segment (start 151.038 101.6) (end 152.3662 100.2718) (width 0.25) (layer "F.Cu") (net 7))
 (segment (start 124.4738 109.0471) (end 131.9663 101.5546) (width 0.25) (layer "F.Cu") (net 7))
 (segment (start 150.9598 91.3589) (end 150.0882 91.3589) (width 0.25) (layer "F.Cu") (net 7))
 (segment (start 144.9116 102.5554) (end 145.867 101.6) (width 0.25) (layer "F.Cu") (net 7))
 (segment (start 152.3662 92.7653) (end 150.9598 91.3589) (width 0.25) (layer "F.Cu") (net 7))
 (segment (start 148.082 90.17) (end 149.2709 90.17) (width 0.25) (layer "F.Cu") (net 7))
 (segment (start 151.0478 104.14) (end 152.8166 102.3712) (width 0.25) (layer "F.Cu") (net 6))
 (segment (start 152.8166 102.3712) (end 152.8166 90.5989) (width 0.25) (layer "F.Cu") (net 6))
 (segment (start 150.1887 104.14) (end 151.0478 104.14) (width 0.25) (layer "F.Cu") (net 6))
 (segment (start 141.441 117.2931) (end 142.24 116.4941) (width 0.25) (layer "F.Cu") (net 6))
 (segment (start 152.8166 90.5989) (end 151.0366 88.8189) (width 0.25) (layer "F.Cu") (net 6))
 (segment (start 124.6419 115.3978) (end 126.5372 117.2931) (width 0.25) (layer "F.Cu") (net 6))
 (segment (start 123.453 113.9649) (end 124.3447 113.9649) (width 0.25) (layer "F.Cu") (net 6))
 (segment (start 149.433 108.4928) (end 149.433 104.8957) (width 0.25) (layer "F.Cu") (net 6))
 (segment (start 151.0366 88.8189) (end 150.0882 88.8189) (width 0.25) (layer "F.Cu") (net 6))
 (segment (start 126.5372 117.2931) (end 141.441 117.2931) (width 0.25) (layer "F.Cu") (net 6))
 (segment (start 142.24 116.4941) (end 142.24 115.6858) (width 0.25) (layer "F.Cu") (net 6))
 (segment (start 149.2709 88.0016) (end 149.2709 87.63) (width 0.25) (layer "F.Cu") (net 6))
 (segment (start 149.433 104.8957) (end 150.1887 104.14) (width 0.25) (layer "F.Cu") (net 6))
 (segment (start 124.3447 113.9649) (end 124.6419 114.2621) (width 0.25) (layer "F.Cu") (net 6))
 (segment (start 123.453 112.776) (end 123.453 113.9649) (width 0.25) (layer "F.Cu") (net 6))
 (segment (start 124.6419 114.2621) (end 124.6419 115.3978) (width 0.25) (layer "F.Cu") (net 6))
 (segment (start 142.24 115.6858) (end 149.433 108.4928) (width 0.25) (layer "F.Cu") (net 6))
 (segment (start 148.082 87.63) (end 149.2709 87.63) (width 0.25) (layer "F.Cu") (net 6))
 (segment (start 150.0882 88.8189) (end 149.2709 88.0016) (width 0.25) (layer "F.Cu") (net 6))
 (segment (start 146.3699 87.6195) (end 142.5105 83.7601) (width 0.25) (layer "B.Cu") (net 5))
 (segment (start 147.7105 86.2789) (end 148.082 86.2789) (width 0.25) (layer "B.Cu") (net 5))
 (segment (start 124.6419 115.316) (end 124.6419 115.3903) (width 0.25) (layer "B.Cu") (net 5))
 (segment (start 128.8899 83.7601) (end 127.249 85.401) (width 0.25) (layer "B.Cu") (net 5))
 (segment (start 124.6419 115.3903) (end 126.9683 117.7167) (width 0.25) (layer "B.Cu") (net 5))
 (segment (start 142.5105 83.7601) (end 128.8899 83.7601) (width 0.25) (layer "B.Cu") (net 5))
 (segment (start 141.8713 117.7167) (end 143.51 116.078) (width 0.25) (layer "B.Cu") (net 5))
 (segment (start 126.9683 117.7167) (end 141.8713 117.7167) (width 0.25) (layer "B.Cu") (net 5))
 (segment (start 146.3699 87.6195) (end 147.7105 86.2789) (width 0.25) (layer "B.Cu") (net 5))
 (segment (start 123.453 115.316) (end 124.6419 115.316) (width 0.25) (layer "B.Cu") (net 5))
 (segment (start 143.51 90.4794) (end 143.51 114.9027) (width 0.25) (layer "B.Cu") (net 5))
 (segment (start 146.3699 87.6195) (end 143.51 90.4794) (width 0.25) (layer "B.Cu") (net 5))
 (segment (start 143.51 116.078) (end 143.51 114.9027) (width 0.25) (layer "B.Cu") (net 5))
 (segment (start 148.082 85.09) (end 148.082 86.2789) (width 0.25) (layer "B.Cu") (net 5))
 (segment (start 144.5422 86.2789) (end 143.6643 85.401) (width 0.25) (layer "F.Cu") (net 2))
 (segment (start 149.1359 86.2789) (end 144.5422 86.2789) (width 0.25) (layer "F.Cu") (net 2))
 (segment (start 142.489 85.401) (end 143.6643 85.401) (width 0.25) (layer "F.Cu") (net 2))
 (segment (start 149.4331 85.9817) (end 149.1359 86.2789) (width 0.25) (layer "F.Cu") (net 2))
 (segment (start 149.4331 85.09) (end 149.4331 85.9817) (width 0.25) (layer "F.Cu") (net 2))
 (segment (start 150.622 85.09) (end 149.4331 85.09) (width 0.25) (layer "F.Cu") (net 2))
 (segment (start 142.24 86.8253) (end 142.24 116.5114) (width 0.25) (layer "B.Cu") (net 2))
 (segment (start 142.24 116.5114) (end 141.498 117.2534) (width 0.25) (layer "B.Cu") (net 2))
 (segment (start 141.498 117.2534) (end 130.7154 117.2534) (width 0.25) (layer "B.Cu") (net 2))
 (segment (start 142.489 86.5763) (end 142.24 86.8253) (width 0.25) (layer "B.Cu") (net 2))
 (segment (start 142.489 85.401) (end 142.489 86.5763) (width 0.25) (layer "B.Cu") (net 2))
 (segment (start 130.7154 117.2534) (end 129.54 116.078) (width 0.25) (layer "B.Cu") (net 2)))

